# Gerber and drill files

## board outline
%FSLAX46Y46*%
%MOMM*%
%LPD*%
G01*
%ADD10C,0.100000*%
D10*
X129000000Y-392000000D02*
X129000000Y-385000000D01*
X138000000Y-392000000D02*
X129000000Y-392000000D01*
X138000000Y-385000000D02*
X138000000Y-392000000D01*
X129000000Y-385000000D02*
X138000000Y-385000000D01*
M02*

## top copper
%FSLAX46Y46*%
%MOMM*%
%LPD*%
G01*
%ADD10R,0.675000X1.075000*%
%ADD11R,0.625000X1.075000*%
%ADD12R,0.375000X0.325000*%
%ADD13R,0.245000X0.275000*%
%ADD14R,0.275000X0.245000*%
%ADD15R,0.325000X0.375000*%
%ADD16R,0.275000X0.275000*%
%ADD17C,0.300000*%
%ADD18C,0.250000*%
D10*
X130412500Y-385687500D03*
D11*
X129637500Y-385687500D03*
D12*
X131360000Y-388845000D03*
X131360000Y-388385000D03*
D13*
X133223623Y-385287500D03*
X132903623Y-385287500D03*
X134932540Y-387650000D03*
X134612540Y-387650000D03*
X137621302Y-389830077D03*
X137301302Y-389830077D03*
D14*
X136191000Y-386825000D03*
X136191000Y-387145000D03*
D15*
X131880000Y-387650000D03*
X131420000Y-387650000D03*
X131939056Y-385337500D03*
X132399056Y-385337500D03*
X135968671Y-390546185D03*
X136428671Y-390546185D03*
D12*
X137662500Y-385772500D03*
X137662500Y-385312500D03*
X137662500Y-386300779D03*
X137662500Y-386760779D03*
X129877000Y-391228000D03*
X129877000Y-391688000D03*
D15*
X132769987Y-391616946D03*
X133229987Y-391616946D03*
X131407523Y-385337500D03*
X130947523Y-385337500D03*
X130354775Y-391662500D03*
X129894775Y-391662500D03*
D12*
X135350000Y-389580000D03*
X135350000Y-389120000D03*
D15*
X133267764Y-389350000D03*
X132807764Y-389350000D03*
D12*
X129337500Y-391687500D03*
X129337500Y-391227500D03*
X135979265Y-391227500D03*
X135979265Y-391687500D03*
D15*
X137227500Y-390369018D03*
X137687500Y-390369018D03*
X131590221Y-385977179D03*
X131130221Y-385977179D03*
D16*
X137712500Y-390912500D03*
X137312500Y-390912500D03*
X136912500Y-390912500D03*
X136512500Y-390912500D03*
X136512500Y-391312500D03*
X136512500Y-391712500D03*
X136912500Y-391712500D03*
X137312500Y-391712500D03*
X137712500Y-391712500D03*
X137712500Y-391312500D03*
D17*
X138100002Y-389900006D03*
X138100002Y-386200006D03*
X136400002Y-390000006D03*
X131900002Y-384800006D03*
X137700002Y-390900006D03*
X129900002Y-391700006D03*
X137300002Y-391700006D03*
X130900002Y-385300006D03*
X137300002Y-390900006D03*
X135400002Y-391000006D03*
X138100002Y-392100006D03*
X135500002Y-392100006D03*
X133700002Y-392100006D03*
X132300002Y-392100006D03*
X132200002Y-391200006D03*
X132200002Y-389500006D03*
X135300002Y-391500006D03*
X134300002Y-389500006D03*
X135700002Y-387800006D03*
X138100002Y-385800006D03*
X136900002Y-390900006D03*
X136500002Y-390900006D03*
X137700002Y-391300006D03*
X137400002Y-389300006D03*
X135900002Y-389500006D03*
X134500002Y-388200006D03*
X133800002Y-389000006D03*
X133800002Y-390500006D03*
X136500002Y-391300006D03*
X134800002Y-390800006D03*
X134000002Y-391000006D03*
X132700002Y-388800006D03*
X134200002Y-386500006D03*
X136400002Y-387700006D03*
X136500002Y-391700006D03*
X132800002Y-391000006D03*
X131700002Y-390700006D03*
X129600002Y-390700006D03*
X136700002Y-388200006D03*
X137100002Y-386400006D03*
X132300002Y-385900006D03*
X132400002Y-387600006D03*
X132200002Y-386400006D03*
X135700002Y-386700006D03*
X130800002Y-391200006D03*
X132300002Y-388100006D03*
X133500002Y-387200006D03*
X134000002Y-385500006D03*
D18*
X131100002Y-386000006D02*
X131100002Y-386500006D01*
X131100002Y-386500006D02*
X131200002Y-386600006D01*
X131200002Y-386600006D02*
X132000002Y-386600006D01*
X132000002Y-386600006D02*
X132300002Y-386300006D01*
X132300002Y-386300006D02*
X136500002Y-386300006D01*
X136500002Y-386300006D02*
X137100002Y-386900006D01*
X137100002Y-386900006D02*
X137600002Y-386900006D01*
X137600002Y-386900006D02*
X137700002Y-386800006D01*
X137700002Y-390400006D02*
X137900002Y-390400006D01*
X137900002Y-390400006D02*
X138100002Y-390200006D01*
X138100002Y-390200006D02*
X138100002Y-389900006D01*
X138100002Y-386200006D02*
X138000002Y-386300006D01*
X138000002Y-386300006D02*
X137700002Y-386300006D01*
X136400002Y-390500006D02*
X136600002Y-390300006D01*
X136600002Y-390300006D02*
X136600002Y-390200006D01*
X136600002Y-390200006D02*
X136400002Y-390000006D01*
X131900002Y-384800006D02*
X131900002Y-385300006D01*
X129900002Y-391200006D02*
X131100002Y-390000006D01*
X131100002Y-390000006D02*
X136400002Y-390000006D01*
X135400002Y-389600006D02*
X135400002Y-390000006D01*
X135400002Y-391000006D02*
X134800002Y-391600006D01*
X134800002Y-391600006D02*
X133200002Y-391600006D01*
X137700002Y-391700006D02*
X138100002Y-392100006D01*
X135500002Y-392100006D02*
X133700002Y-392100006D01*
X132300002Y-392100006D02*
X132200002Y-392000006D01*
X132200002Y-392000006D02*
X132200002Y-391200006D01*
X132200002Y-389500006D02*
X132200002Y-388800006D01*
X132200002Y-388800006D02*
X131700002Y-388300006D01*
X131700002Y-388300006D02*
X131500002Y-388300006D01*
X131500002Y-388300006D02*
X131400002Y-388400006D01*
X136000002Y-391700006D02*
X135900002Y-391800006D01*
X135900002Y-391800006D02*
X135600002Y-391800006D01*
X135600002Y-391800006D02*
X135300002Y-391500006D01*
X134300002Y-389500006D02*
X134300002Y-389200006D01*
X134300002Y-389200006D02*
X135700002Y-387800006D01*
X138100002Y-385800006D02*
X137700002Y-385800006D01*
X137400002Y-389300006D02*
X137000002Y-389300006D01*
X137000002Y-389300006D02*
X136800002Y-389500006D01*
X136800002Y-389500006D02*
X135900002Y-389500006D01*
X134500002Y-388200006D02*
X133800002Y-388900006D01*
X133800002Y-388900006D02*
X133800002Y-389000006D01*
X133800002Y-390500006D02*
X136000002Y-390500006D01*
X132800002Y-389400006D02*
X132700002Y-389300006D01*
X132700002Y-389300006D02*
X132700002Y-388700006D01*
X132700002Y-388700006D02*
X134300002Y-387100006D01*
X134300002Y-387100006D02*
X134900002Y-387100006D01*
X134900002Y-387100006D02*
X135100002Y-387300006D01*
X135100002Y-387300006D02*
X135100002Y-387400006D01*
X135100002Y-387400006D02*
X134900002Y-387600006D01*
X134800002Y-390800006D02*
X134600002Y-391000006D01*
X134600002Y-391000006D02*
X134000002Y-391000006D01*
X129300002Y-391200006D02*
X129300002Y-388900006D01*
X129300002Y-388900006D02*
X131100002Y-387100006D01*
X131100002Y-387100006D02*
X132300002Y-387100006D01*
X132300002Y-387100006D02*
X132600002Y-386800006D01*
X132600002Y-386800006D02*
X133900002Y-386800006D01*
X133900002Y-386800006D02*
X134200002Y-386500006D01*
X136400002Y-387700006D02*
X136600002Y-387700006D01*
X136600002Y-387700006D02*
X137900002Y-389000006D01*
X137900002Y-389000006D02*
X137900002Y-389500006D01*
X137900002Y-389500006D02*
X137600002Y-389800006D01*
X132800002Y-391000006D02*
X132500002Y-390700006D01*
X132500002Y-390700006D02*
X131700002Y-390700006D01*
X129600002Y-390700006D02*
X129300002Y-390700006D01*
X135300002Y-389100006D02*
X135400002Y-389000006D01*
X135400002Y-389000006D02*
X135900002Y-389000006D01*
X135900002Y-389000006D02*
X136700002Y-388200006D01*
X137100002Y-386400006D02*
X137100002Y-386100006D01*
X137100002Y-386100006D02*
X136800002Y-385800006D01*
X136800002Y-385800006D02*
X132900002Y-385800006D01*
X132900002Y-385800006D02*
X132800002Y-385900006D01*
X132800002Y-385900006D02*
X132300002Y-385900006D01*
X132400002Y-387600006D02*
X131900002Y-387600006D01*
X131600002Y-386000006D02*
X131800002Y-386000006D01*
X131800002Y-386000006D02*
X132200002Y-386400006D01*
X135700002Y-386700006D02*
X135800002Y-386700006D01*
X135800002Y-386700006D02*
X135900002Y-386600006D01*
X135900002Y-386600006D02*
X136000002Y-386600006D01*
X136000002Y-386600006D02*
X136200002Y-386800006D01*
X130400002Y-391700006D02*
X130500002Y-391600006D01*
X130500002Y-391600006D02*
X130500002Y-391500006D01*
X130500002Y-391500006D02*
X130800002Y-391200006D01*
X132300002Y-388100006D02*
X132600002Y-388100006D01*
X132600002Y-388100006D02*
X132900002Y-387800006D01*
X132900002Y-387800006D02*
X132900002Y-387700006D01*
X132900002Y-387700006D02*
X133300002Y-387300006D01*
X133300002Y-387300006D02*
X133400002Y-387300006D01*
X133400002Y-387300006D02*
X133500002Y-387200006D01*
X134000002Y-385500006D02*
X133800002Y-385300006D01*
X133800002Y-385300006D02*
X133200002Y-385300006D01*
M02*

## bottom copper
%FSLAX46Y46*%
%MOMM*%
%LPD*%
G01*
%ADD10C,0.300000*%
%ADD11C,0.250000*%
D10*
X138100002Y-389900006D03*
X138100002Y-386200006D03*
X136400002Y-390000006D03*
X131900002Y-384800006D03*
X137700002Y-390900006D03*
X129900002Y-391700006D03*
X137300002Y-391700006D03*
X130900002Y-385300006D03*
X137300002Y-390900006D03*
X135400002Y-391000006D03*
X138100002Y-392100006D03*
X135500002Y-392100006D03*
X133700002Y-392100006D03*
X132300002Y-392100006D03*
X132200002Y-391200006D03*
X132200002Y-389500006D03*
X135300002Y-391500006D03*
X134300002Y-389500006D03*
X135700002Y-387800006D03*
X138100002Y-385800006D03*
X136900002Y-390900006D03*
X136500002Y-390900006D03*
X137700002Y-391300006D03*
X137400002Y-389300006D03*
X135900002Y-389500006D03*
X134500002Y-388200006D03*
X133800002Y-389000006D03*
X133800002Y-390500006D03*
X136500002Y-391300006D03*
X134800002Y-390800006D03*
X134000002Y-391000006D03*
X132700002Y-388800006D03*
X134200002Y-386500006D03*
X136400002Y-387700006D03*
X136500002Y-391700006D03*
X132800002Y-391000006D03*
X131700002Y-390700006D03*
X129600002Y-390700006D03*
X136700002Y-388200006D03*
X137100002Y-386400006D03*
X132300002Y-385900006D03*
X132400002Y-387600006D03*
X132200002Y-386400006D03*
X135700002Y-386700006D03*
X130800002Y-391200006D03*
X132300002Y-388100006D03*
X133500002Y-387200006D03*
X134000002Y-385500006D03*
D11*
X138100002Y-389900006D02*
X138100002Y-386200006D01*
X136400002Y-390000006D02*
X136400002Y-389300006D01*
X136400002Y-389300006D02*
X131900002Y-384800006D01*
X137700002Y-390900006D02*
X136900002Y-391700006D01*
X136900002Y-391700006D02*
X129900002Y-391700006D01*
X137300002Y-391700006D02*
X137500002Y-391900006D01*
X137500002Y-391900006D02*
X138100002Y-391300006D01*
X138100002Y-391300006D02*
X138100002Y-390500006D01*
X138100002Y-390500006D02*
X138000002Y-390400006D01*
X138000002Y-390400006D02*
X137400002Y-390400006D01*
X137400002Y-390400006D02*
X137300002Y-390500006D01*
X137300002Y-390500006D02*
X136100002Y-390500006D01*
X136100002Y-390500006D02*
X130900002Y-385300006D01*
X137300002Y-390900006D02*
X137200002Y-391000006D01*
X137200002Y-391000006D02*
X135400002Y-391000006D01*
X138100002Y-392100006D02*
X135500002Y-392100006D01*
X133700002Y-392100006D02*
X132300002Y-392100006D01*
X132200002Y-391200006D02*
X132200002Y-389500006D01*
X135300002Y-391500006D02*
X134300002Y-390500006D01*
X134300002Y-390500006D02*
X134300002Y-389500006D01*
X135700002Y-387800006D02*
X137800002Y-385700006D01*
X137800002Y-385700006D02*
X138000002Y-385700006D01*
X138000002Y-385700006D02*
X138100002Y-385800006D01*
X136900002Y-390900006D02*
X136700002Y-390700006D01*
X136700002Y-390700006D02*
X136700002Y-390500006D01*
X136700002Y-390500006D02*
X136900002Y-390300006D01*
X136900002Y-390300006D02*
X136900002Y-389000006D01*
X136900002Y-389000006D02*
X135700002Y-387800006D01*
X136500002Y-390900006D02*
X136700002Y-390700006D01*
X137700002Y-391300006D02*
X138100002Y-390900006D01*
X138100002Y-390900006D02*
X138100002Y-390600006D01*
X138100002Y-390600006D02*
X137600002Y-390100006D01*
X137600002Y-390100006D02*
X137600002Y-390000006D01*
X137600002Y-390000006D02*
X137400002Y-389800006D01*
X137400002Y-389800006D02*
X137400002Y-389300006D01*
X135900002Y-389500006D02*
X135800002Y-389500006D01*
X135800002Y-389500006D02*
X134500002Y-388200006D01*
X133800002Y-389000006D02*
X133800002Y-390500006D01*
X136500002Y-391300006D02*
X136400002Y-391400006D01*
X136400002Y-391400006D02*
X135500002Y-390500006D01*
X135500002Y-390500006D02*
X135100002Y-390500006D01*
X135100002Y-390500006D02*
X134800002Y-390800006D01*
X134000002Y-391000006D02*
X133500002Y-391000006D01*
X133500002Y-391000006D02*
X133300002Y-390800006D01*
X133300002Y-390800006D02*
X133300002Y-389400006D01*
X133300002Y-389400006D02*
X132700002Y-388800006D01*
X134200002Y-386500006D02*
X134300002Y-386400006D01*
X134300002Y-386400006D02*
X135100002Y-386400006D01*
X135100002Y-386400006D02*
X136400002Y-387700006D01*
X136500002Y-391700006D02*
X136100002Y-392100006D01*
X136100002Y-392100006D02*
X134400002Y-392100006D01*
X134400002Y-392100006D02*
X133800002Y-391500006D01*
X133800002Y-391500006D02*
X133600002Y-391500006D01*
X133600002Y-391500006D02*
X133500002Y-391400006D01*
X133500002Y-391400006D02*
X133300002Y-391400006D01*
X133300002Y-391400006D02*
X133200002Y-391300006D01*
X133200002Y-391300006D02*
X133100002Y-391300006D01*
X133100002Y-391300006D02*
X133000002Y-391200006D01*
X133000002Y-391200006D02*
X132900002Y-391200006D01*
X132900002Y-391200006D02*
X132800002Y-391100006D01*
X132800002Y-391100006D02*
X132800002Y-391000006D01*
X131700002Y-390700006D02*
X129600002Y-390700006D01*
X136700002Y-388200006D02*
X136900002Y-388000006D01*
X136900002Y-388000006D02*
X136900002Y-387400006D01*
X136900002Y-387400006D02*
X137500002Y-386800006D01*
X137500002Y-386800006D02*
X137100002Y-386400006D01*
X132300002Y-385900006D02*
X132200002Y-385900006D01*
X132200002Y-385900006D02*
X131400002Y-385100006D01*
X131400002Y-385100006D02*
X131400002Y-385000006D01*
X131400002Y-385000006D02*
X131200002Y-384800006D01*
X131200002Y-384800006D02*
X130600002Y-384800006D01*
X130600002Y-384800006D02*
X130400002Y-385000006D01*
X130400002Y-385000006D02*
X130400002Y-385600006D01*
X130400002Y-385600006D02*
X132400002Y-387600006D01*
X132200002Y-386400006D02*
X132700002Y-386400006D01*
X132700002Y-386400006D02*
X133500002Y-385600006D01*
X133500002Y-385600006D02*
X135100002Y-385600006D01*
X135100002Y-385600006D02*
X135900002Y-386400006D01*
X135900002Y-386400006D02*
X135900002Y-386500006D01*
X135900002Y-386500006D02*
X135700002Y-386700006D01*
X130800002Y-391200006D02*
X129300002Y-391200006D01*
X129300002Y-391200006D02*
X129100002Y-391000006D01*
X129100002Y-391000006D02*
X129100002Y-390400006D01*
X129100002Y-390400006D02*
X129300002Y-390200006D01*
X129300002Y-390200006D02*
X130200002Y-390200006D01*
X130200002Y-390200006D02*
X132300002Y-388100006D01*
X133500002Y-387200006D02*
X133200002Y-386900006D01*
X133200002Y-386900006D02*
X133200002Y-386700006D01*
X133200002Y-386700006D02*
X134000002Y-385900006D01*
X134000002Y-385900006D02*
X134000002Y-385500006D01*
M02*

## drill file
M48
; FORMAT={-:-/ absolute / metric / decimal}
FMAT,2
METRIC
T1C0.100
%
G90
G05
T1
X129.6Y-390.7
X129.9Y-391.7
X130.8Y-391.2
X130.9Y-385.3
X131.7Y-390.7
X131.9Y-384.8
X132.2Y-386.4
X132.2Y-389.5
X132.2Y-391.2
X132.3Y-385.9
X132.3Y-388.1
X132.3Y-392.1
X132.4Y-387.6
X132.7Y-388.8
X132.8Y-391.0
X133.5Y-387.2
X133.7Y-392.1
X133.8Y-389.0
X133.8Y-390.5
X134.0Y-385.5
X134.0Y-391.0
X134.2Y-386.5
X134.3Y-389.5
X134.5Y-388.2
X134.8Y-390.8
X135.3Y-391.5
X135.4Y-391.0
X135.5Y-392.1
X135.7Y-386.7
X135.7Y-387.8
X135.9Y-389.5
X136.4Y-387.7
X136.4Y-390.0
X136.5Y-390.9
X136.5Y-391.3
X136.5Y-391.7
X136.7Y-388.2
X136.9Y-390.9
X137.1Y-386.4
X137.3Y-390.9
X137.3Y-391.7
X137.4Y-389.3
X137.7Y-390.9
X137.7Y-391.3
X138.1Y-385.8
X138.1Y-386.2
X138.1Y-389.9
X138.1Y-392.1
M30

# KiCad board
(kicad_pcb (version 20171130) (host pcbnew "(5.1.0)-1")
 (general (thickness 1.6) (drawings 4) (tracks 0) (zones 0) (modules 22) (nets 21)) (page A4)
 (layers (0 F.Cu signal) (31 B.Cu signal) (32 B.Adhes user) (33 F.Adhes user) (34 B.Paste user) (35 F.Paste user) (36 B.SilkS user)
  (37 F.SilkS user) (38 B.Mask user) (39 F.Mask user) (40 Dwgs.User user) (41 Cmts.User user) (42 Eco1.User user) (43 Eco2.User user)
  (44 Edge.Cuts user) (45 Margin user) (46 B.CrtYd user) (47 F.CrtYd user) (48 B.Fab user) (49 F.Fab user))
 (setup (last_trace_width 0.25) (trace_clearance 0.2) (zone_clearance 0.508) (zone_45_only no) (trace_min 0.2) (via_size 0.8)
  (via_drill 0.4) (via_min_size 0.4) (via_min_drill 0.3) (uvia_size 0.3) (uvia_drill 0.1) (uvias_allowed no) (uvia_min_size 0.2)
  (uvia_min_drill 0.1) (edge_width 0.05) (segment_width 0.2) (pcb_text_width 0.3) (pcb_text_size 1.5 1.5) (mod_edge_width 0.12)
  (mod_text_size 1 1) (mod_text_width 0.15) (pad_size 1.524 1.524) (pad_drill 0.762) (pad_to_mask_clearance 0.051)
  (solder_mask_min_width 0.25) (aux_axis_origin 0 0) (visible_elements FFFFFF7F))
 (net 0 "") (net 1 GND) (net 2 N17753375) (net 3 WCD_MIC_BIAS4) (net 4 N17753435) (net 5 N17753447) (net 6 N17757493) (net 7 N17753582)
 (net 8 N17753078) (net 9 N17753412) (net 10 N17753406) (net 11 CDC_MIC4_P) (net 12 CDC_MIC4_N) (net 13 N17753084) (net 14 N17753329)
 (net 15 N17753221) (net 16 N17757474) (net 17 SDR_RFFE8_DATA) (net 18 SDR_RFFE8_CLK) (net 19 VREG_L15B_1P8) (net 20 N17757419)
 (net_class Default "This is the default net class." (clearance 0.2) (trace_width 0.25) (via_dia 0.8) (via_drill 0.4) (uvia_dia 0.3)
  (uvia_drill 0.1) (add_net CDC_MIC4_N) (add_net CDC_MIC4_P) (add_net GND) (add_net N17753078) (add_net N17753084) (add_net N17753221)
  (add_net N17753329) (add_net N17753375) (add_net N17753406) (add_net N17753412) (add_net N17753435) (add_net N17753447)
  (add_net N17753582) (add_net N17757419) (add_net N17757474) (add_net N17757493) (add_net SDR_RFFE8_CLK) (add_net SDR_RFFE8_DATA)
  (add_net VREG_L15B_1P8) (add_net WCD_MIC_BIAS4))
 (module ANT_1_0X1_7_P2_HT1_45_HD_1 (layer F.Cu) (at 129.862500 385.687500 270.000000)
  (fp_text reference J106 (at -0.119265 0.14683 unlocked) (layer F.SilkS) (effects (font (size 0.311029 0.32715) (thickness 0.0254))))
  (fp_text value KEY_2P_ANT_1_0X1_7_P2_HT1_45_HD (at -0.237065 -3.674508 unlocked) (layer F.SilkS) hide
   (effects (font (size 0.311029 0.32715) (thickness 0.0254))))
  (pad 1 smd rect (at 0 -0.55) (size 0.675 1.075) (layers F.Cu F.Mask F.Paste) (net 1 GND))
  (pad 2 smd rect (at 0 0.225) (size 0.625 1.075) (layers F.Cu F.Mask F.Paste) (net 1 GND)))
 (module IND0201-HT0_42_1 (layer F.Cu) (at 131.360000 388.615000 90.000000)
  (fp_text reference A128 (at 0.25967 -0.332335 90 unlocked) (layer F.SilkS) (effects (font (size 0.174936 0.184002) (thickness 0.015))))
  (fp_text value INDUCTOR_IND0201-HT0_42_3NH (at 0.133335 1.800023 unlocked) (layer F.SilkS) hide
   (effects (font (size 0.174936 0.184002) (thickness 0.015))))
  (pad 1 smd rect (at -0.23 0) (size 0.375 0.325) (layers F.Cu F.Mask F.Paste) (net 1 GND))
  (pad 2 smd rect (at 0.23 0) (size 0.375 0.325) (layers F.Cu F.Mask F.Paste) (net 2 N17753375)))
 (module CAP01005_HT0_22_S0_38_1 (layer F.Cu) (at 133.063623 385.287500 180.000000)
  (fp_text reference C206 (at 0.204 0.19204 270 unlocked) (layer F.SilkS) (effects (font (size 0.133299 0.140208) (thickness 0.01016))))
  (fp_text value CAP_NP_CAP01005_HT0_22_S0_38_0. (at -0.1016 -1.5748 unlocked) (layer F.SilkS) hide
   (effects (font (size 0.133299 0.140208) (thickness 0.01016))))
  (pad 1 smd rect (at -0.16 0 270.000000) (size 0.275 0.245) (layers F.Cu F.Mask F.Paste) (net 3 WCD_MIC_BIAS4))
  (pad 2 smd rect (at 0.16 0 270.000000) (size 0.275 0.245) (layers F.Cu F.Mask F.Paste) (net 1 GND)))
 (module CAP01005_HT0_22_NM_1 (layer F.Cu) (at 134.772540 387.650000 180.000000)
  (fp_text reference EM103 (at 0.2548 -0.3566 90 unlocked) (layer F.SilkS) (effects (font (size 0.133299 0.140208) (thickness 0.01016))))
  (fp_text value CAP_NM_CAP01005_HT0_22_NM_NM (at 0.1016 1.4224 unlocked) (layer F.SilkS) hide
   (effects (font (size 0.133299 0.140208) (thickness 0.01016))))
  (pad 1 smd rect (at -0.16 0 90.000000) (size 0.275 0.245) (layers F.Cu F.Mask F.Paste) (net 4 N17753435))
  (pad 2 smd rect (at 0.16 0 90.000000) (size 0.275 0.245) (layers F.Cu F.Mask F.Paste) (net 1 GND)))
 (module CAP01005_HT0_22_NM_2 (layer F.Cu) (at 137.461302 389.830077 180.000000)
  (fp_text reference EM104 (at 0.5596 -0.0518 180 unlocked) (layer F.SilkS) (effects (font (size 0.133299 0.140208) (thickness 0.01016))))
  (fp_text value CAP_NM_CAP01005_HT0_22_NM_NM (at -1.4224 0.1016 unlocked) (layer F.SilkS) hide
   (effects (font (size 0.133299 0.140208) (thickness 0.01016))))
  (pad 1 smd rect (at -0.16 0) (size 0.245 0.275) (layers F.Cu F.Mask F.Paste) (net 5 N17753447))
  (pad 2 smd rect (at 0.16 0) (size 0.245 0.275) (layers F.Cu F.Mask F.Paste) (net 1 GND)))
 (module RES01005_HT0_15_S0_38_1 (layer F.Cu) (at 136.191000 386.985000 270.000000)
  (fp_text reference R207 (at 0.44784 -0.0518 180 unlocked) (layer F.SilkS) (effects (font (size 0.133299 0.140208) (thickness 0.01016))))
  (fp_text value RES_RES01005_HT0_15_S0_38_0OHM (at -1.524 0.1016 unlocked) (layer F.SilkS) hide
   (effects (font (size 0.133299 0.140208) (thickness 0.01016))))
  (pad 1 smd rect (at -0.16 0 90.000000) (size 0.245 0.275) (layers F.Cu F.Mask F.Paste) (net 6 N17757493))
  (pad 2 smd rect (at 0.16 0 90.000000) (size 0.245 0.275) (layers F.Cu F.Mask F.Paste) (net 1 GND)))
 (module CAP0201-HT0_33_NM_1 (layer F.Cu) (at 131.650000 387.650000 180.000000)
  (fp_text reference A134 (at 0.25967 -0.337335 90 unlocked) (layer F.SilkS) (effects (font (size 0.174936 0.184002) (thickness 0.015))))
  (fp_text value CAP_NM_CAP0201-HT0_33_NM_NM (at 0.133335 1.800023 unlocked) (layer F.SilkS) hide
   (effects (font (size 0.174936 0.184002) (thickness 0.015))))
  (pad 1 smd rect (at -0.23 0 90.000000) (size 0.375 0.325) (layers F.Cu F.Mask F.Paste) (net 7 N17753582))
  (pad 2 smd rect (at 0.23 0 90.000000) (size 0.375 0.325) (layers F.Cu F.Mask F.Paste) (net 1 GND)))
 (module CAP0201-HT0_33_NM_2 (layer F.Cu) (at 132.169056 385.337500)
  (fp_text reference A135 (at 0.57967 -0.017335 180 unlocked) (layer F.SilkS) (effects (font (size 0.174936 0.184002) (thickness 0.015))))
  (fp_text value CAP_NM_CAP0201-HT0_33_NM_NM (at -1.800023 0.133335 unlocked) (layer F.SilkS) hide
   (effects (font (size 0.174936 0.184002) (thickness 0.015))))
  (pad 1 smd rect (at -0.23 0 180.000000) (size 0.325 0.375) (layers F.Cu F.Mask F.Paste) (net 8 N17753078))
  (pad 2 smd rect (at 0.23 0 180.000000) (size 0.325 0.375) (layers F.Cu F.Mask F.Paste) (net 1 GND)))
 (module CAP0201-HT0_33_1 (layer F.Cu) (at 136.198671 390.546185)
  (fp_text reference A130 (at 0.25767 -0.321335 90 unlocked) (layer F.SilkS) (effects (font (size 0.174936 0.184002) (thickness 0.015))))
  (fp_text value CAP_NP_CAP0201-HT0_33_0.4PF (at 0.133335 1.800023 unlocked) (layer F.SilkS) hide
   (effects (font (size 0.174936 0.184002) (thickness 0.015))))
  (pad 1 smd rect (at -0.23 0 270.000000) (size 0.375 0.325) (layers F.Cu F.Mask F.Paste) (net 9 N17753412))
  (pad 2 smd rect (at 0.23 0 270.000000) (size 0.375 0.325) (layers F.Cu F.Mask F.Paste) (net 8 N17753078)))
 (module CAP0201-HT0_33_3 (layer F.Cu) (at 137.662500 385.542500 90.000000)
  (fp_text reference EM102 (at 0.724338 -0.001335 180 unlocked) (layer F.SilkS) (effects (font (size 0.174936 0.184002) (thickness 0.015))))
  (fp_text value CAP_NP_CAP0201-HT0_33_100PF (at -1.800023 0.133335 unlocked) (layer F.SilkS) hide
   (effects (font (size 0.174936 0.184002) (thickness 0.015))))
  (pad 1 smd rect (at -0.23 0 270.000000) (size 0.325 0.375) (layers F.Cu F.Mask F.Paste) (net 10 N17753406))
  (pad 2 smd rect (at 0.23 0 270.000000) (size 0.325 0.375) (layers F.Cu F.Mask F.Paste) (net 1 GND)))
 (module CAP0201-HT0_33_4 (layer F.Cu) (at 137.662500 386.530779 270.000000)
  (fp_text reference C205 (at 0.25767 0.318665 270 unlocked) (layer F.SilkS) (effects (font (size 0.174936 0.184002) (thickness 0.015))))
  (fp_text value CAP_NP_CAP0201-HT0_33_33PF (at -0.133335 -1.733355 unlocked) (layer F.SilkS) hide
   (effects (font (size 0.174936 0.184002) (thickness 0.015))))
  (pad 1 smd rect (at -0.23 0) (size 0.375 0.325) (layers F.Cu F.Mask F.Paste) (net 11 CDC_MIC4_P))
  (pad 2 smd rect (at 0.23 0) (size 0.375 0.325) (layers F.Cu F.Mask F.Paste) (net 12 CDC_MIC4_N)))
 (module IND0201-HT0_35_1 (layer F.Cu) (at 129.877000 391.458000 270.000000)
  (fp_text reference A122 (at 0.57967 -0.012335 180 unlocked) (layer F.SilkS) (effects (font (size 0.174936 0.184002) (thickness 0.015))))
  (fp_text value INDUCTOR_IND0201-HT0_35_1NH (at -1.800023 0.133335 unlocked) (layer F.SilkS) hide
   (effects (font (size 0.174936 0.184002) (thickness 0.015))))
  (pad 1 smd rect (at -0.23 0 90.000000) (size 0.325 0.375) (layers F.Cu F.Mask F.Paste) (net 8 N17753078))
  (pad 2 smd rect (at 0.23 0 90.000000) (size 0.325 0.375) (layers F.Cu F.Mask F.Paste) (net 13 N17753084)))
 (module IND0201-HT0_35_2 (layer F.Cu) (at 132.999987 391.616946)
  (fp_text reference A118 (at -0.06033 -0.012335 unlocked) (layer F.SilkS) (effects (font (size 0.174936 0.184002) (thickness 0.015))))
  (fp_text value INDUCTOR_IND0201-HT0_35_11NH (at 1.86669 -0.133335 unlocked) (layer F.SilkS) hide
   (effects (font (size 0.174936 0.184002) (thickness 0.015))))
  (pad 1 smd rect (at -0.23 0) (size 0.325 0.375) (layers F.Cu F.Mask F.Paste) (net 1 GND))
  (pad 2 smd rect (at 0.23 0) (size 0.325 0.375) (layers F.Cu F.Mask F.Paste) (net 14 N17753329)))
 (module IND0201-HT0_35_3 (layer F.Cu) (at 131.177523 385.337500 180.000000)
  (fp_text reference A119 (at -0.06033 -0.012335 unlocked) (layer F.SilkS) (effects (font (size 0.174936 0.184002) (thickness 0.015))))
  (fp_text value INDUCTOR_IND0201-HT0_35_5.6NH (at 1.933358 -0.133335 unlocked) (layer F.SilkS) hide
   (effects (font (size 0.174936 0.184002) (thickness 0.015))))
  (pad 1 smd rect (at -0.23 0 180.000000) (size 0.325 0.375) (layers F.Cu F.Mask F.Paste) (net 1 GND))
  (pad 2 smd rect (at 0.23 0 180.000000) (size 0.325 0.375) (layers F.Cu F.Mask F.Paste) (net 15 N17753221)))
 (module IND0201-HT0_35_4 (layer F.Cu) (at 130.124775 391.662500 180.000000)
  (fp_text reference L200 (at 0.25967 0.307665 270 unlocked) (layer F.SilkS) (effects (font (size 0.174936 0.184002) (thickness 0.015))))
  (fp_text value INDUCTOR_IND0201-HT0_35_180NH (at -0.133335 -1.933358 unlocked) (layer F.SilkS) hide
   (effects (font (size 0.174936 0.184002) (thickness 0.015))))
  (pad 1 smd rect (at -0.23 0 270.000000) (size 0.375 0.325) (layers F.Cu F.Mask F.Paste) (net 3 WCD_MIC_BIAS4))
  (pad 2 smd rect (at 0.23 0 270.000000) (size 0.375 0.325) (layers F.Cu F.Mask F.Paste) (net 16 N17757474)))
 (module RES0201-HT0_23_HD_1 (layer F.Cu) (at 135.350000 389.350000 90.000000)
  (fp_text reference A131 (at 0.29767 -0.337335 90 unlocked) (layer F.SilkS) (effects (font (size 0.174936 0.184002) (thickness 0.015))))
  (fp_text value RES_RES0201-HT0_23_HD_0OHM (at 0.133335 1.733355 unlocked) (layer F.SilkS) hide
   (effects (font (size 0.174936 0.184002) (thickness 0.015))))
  (pad 1 smd rect (at -0.23 0) (size 0.375 0.325) (layers F.Cu F.Mask F.Paste) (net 8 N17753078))
  (pad 2 smd rect (at 0.23 0) (size 0.375 0.325) (layers F.Cu F.Mask F.Paste) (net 7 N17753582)))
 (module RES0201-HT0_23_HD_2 (layer F.Cu) (at 133.037764 389.350000 180.000000)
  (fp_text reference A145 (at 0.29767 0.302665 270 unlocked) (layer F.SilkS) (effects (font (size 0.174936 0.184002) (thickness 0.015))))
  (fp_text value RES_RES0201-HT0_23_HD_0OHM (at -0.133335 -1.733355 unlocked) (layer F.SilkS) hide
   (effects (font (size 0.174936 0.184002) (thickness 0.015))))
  (pad 1 smd rect (at -0.23 0 270.000000) (size 0.375 0.325) (layers F.Cu F.Mask F.Paste) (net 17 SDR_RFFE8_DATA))
  (pad 2 smd rect (at 0.23 0 270.000000) (size 0.375 0.325) (layers F.Cu F.Mask F.Paste) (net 4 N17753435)))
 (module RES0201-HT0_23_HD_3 (layer F.Cu) (at 129.337500 391.457500 90.000000)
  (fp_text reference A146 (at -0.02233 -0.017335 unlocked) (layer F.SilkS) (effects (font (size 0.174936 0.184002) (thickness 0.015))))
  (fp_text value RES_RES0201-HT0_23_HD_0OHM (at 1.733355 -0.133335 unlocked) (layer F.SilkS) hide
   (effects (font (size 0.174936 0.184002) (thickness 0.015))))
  (pad 1 smd rect (at -0.23 0 90.000000) (size 0.325 0.375) (layers F.Cu F.Mask F.Paste) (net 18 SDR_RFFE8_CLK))
  (pad 2 smd rect (at 0.23 0 90.000000) (size 0.325 0.375) (layers F.Cu F.Mask F.Paste) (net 5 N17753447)))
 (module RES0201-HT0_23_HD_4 (layer F.Cu) (at 135.979265 391.457500 270.000000)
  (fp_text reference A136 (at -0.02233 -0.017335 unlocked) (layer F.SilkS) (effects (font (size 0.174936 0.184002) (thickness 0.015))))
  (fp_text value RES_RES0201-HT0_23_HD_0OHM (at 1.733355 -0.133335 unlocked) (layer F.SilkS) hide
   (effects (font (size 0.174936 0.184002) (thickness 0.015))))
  (pad 1 smd rect (at -0.23 0 270.000000) (size 0.325 0.375) (layers F.Cu F.Mask F.Paste) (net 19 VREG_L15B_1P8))
  (pad 2 smd rect (at 0.23 0 270.000000) (size 0.325 0.375) (layers F.Cu F.Mask F.Paste) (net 10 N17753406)))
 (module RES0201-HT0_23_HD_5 (layer F.Cu) (at 137.457500 390.369018)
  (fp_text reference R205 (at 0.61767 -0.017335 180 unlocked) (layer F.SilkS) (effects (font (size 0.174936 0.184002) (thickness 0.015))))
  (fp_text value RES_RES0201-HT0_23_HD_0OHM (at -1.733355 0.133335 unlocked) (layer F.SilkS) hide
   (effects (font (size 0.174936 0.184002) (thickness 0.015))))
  (pad 1 smd rect (at -0.23 0 180.000000) (size 0.325 0.375) (layers F.Cu F.Mask F.Paste) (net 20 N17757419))
  (pad 2 smd rect (at 0.23 0 180.000000) (size 0.325 0.375) (layers F.Cu F.Mask F.Paste) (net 11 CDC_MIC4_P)))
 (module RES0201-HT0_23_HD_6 (layer F.Cu) (at 131.360221 385.977179 180.000000)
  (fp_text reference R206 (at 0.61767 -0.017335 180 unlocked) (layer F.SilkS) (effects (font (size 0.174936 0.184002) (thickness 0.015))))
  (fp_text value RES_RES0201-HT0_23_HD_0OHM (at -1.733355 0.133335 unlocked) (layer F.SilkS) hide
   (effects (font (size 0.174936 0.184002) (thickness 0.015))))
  (pad 1 smd rect (at -0.23 0) (size 0.325 0.375) (layers F.Cu F.Mask F.Paste) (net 6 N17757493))
  (pad 2 smd rect (at 0.23 0) (size 0.325 0.375) (layers F.Cu F.Mask F.Paste) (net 12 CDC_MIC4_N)))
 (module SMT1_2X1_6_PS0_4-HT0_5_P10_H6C (layer F.Cu) (at 137.112500 391.312500 180.000000)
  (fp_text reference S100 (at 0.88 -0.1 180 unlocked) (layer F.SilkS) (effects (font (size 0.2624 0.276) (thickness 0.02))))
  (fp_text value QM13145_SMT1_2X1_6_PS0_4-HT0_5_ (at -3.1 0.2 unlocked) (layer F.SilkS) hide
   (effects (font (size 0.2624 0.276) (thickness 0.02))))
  (pad 1 smd rect (at -0.6 0.4) (size 0.275 0.275) (layers F.Cu F.Mask F.Paste) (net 13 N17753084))
  (pad 2 smd rect (at -0.2 0.4) (size 0.275 0.275) (layers F.Cu F.Mask F.Paste) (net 14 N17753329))
  (pad 3 smd rect (at 0.2 0.4) (size 0.275 0.275) (layers F.Cu F.Mask F.Paste) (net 10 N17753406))
  (pad 4 smd rect (at 0.6 0.4) (size 0.275 0.275) (layers F.Cu F.Mask F.Paste) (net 10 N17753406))
  (pad 5 smd rect (at 0.6 0) (size 0.275 0.275) (layers F.Cu F.Mask F.Paste) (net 4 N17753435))
  (pad 6 smd rect (at 0.6 -0.4) (size 0.275 0.275) (layers F.Cu F.Mask F.Paste) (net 5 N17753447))
  (pad 7 smd rect (at 0.2 -0.4) (size 0.275 0.275) (layers F.Cu F.Mask F.Paste) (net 1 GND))
  (pad 8 smd rect (at -0.2 -0.4) (size 0.275 0.275) (layers F.Cu F.Mask F.Paste) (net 15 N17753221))
  (pad 9 smd rect (at -0.6 -0.4) (size 0.275 0.275) (layers F.Cu F.Mask F.Paste) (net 2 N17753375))
  (pad 10 smd rect (at -0.6 0) (size 0.275 0.275) (layers F.Cu F.Mask F.Paste) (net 9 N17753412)))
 (gr_line (start 129 392) (end 129 385) (layer Edge.Cuts) (width 0.1))
 (gr_line (start 138 392) (end 129 392) (layer Edge.Cuts) (width 0.1))
 (gr_line (start 138 385) (end 138 392) (layer Edge.Cuts) (width 0.1))
 (gr_line (start 129 385) (end 138 385) (layer Edge.Cuts) (width 0.1))
 (segment (start 131.100002 386.000006) (end 131.100002 386.500006) (width 0.250000) (layer F.Cu) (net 12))
 (segment (start 131.100002 386.500006) (end 131.200002 386.600006) (width 0.250000) (layer F.Cu) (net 12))
 (segment (start 131.200002 386.600006) (end 132.000002 386.600006) (width 0.250000) (layer F.Cu) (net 12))
 (segment (start 132.000002 386.600006) (end 132.300002 386.300006) (width 0.250000) (layer F.Cu) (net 12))
 (segment (start 132.300002 386.300006) (end 136.500002 386.300006) (width 0.250000) (layer F.Cu) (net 12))
 (segment (start 136.500002 386.300006) (end 137.100002 386.900006) (width 0.250000) (layer F.Cu) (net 12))
 (segment (start 137.100002 386.900006) (end 137.600002 386.900006) (width 0.250000) (layer F.Cu) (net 12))
 (segment (start 137.600002 386.900006) (end 137.700002 386.800006) (width 0.250000) (layer F.Cu) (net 12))
 (segment (start 137.700002 390.400006) (end 137.900002 390.400006) (width 0.250000) (layer F.Cu) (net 11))
 (segment (start 137.900002 390.400006) (end 138.100002 390.200006) (width 0.250000) (layer F.Cu) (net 11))
 (segment (start 138.100002 390.200006) (end 138.100002 389.900006) (width 0.250000) (layer F.Cu) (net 11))
 (segment (start 138.100002 389.900006) (end 138.100002 386.200006) (width 0.250000) (layer B.Cu) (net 11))
 (segment (start 138.100002 386.200006) (end 138.000002 386.300006) (width 0.250000) (layer F.Cu) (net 11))
 (segment (start 138.000002 386.300006) (end 137.700002 386.300006) (width 0.250000) (layer F.Cu) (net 11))
 (via micro (at 138.100002 389.900006) (size 0.300000) (drill 0.100000) (layers F.Cu B.Cu) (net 11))
 (via micro (at 138.100002 386.200006) (size 0.300000) (drill 0.100000) (layers F.Cu B.Cu) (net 11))
 (segment (start 136.400002 390.500006) (end 136.600002 390.300006) (width 0.250000) (layer F.Cu) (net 8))
 (segment (start 136.600002 390.300006) (end 136.600002 390.200006) (width 0.250000) (layer F.Cu) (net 8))
 (segment (start 136.600002 390.200006) (end 136.400002 390.000006) (width 0.250000) (layer F.Cu) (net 8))
 (segment (start 136.400002 390.000006) (end 136.400002 389.300006) (width 0.250000) (layer B.Cu) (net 8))
 (segment (start 136.400002 389.300006) (end 131.900002 384.800006) (width 0.250000) (layer B.Cu) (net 8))
 (segment (start 131.900002 384.800006) (end 131.900002 385.300006) (width 0.250000) (layer F.Cu) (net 8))
 (segment (start 129.900002 391.200006) (end 131.100002 390.000006) (width 0.250000) (layer F.Cu) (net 8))
 (segment (start 131.100002 390.000006) (end 136.400002 390.000006) (width 0.250000) (layer F.Cu) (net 8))
 (segment (start 135.400002 389.600006) (end 135.400002 390.000006) (width 0.250000) (layer F.Cu) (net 8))
 (via micro (at 136.400002 390.000006) (size 0.300000) (drill 0.100000) (layers F.Cu B.Cu) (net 8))
 (via micro (at 131.900002 384.800006) (size 0.300000) (drill 0.100000) (layers F.Cu B.Cu) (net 8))
 (segment (start 137.700002 390.900006) (end 136.900002 391.700006) (width 0.250000) (layer B.Cu) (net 13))
 (segment (start 136.900002 391.700006) (end 129.900002 391.700006) (width 0.250000) (layer B.Cu) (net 13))
 (via micro (at 137.700002 390.900006) (size 0.300000) (drill 0.100000) (layers F.Cu B.Cu) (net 13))
 (via micro (at 129.900002 391.700006) (size 0.300000) (drill 0.100000) (layers F.Cu B.Cu) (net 13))
 (segment (start 137.300002 391.700006) (end 137.500002 391.900006) (width 0.250000) (layer B.Cu) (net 15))
 (segment (start 137.500002 391.900006) (end 138.100002 391.300006) (width 0.250000) (layer B.Cu) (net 15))
 (segment (start 138.100002 391.300006) (end 138.100002 390.500006) (width 0.250000) (layer B.Cu) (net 15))
 (segment (start 138.100002 390.500006) (end 138.000002 390.400006) (width 0.250000) (layer B.Cu) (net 15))
 (segment (start 138.000002 390.400006) (end 137.400002 390.400006) (width 0.250000) (layer B.Cu) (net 15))
 (segment (start 137.400002 390.400006) (end 137.300002 390.500006) (width 0.250000) (layer B.Cu) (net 15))
 (segment (start 137.300002 390.500006) (end 136.100002 390.500006) (width 0.250000) (layer B.Cu) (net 15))
 (segment (start 136.100002 390.500006) (end 130.900002 385.300006) (width 0.250000) (layer B.Cu) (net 15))
 (via micro (at 137.300002 391.700006) (size 0.300000) (drill 0.100000) (layers F.Cu B.Cu) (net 15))
 (via micro (at 130.900002 385.300006) (size 0.300000) (drill 0.100000) (layers F.Cu B.Cu) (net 15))
 (segment (start 137.300002 390.900006) (end 137.200002 391.000006) (width 0.250000) (layer B.Cu) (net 14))
 (segment (start 137.200002 391.000006) (end 135.400002 391.000006) (width 0.250000) (layer B.Cu) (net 14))
 (segment (start 135.400002 391.000006) (end 134.800002 391.600006) (width 0.250000) (layer F.Cu) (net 14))
 (segment (start 134.800002 391.600006) (end 133.200002 391.600006) (width 0.250000) (layer F.Cu) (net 14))
 (via micro (at 137.300002 390.900006) (size 0.300000) (drill 0.100000) (layers F.Cu B.Cu) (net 14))
 (via micro (at 135.400002 391.000006) (size 0.300000) (drill 0.100000) (layers F.Cu B.Cu) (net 14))
 (segment (start 137.700002 391.700006) (end 138.100002 392.100006) (width 0.250000) (layer F.Cu) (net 2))
 (segment (start 138.100002 392.100006) (end 135.500002 392.100006) (width 0.250000) (layer B.Cu) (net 2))
 (segment (start 135.500002 392.100006) (end 133.700002 392.100006) (width 0.250000) (layer F.Cu) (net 2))
 (segment (start 133.700002 392.100006) (end 132.300002 392.100006) (width 0.250000) (layer B.Cu) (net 2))
 (segment (start 132.300002 392.100006) (end 132.200002 392.000006) (width 0.250000) (layer F.Cu) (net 2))
 (segment (start 132.200002 392.000006) (end 132.200002 391.200006) (width 0.250000) (layer F.Cu) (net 2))
 (segment (start 132.200002 391.200006) (end 132.200002 389.500006) (width 0.250000) (layer B.Cu) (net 2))
 (segment (start 132.200002 389.500006) (end 132.200002 388.800006) (width 0.250000) (layer F.Cu) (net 2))
 (segment (start 132.200002 388.800006) (end 131.700002 388.300006) (width 0.250000) (layer F.Cu) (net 2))
 (segment (start 131.700002 388.300006) (end 131.500002 388.300006) (width 0.250000) (layer F.Cu) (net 2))
 (segment (start 131.500002 388.300006) (end 131.400002 388.400006) (width 0.250000) (layer F.Cu) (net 2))
 (via micro (at 138.100002 392.100006) (size 0.300000) (drill 0.100000) (layers F.Cu B.Cu) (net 2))
 (via micro (at 135.500002 392.100006) (size 0.300000) (drill 0.100000) (layers F.Cu B.Cu) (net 2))
 (via micro (at 133.700002 392.100006) (size 0.300000) (drill 0.100000) (layers F.Cu B.Cu) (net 2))
 (via micro (at 132.300002 392.100006) (size 0.300000) (drill 0.100000) (layers F.Cu B.Cu) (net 2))
 (via micro (at 132.200002 391.200006) (size 0.300000) (drill 0.100000) (layers F.Cu B.Cu) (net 2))
 (via micro (at 132.200002 389.500006) (size 0.300000) (drill 0.100000) (layers F.Cu B.Cu) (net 2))
 (segment (start 136.000002 391.700006) (end 135.900002 391.800006) (width 0.250000) (layer F.Cu) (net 10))
 (segment (start 135.900002 391.800006) (end 135.600002 391.800006) (width 0.250000) (layer F.Cu) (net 10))
 (segment (start 135.600002 391.800006) (end 135.300002 391.500006) (width 0.250000) (layer F.Cu) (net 10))
 (segment (start 135.300002 391.500006) (end 134.300002 390.500006) (width 0.250000) (layer B.Cu) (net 10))
 (segment (start 134.300002 390.500006) (end 134.300002 389.500006) (width 0.250000) (layer B.Cu) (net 10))
 (segment (start 134.300002 389.500006) (end 134.300002 389.200006) (width 0.250000) (layer F.Cu) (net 10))
 (segment (start 134.300002 389.200006) (end 135.700002 387.800006) (width 0.250000) (layer F.Cu) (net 10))
 (segment (start 135.700002 387.800006) (end 137.800002 385.700006) (width 0.250000) (layer B.Cu) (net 10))
 (segment (start 137.800002 385.700006) (end 138.000002 385.700006) (width 0.250000) (layer B.Cu) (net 10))
 (segment (start 138.000002 385.700006) (end 138.100002 385.800006) (width 0.250000) (layer B.Cu) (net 10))
 (segment (start 138.100002 385.800006) (end 137.700002 385.800006) (width 0.250000) (layer F.Cu) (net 10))
 (segment (start 136.900002 390.900006) (end 136.700002 390.700006) (width 0.250000) (layer B.Cu) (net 10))
 (segment (start 136.700002 390.700006) (end 136.700002 390.500006) (width 0.250000) (layer B.Cu) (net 10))
 (segment (start 136.700002 390.500006) (end 136.900002 390.300006) (width 0.250000) (layer B.Cu) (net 10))
 (segment (start 136.900002 390.300006) (end 136.900002 389.000006) (width 0.250000) (layer B.Cu) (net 10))
 (segment (start 136.900002 389.000006) (end 135.700002 387.800006) (width 0.250000) (layer B.Cu) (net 10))
 (segment (start 136.500002 390.900006) (end 136.700002 390.700006) (width 0.250000) (layer B.Cu) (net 10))
 (via micro (at 135.300002 391.500006) (size 0.300000) (drill 0.100000) (layers F.Cu B.Cu) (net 10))
 (via micro (at 134.300002 389.500006) (size 0.300000) (drill 0.100000) (layers F.Cu B.Cu) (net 10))
 (via micro (at 135.700002 387.800006) (size 0.300000) (drill 0.100000) (layers F.Cu B.Cu) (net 10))
 (via micro (at 138.100002 385.800006) (size 0.300000) (drill 0.100000) (layers F.Cu B.Cu) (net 10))
 (via micro (at 136.900002 390.900006) (size 0.300000) (drill 0.100000) (layers F.Cu B.Cu) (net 10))
 (via micro (at 136.500002 390.900006) (size 0.300000) (drill 0.100000) (layers F.Cu B.Cu) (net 10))
 (segment (start 137.700002 391.300006) (end 138.100002 390.900006) (width 0.250000) (layer B.Cu) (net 9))
 (segment (start 138.100002 390.900006) (end 138.100002 390.600006) (width 0.250000) (layer B.Cu) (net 9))
 (segment (start 138.100002 390.600006) (end 137.600002 390.100006) (width 0.250000) (layer B.Cu) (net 9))
 (segment (start 137.600002 390.100006) (end 137.600002 390.000006) (width 0.250000) (layer B.Cu) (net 9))
 (segment (start 137.600002 390.000006) (end 137.400002 389.800006) (width 0.250000) (layer B.Cu) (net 9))
 (segment (start 137.400002 389.800006) (end 137.400002 389.300006) (width 0.250000) (layer B.Cu) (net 9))
 (segment (start 137.400002 389.300006) (end 137.000002 389.300006) (width 0.250000) (layer F.Cu) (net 9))
 (segment (start 137.000002 389.300006) (end 136.800002 389.500006) (width 0.250000) (layer F.Cu) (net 9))
 (segment (start 136.800002 389.500006) (end 135.900002 389.500006) (width 0.250000) (layer F.Cu) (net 9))
 (segment (start 135.900002 389.500006) (end 135.800002 389.500006) (width 0.250000) (layer B.Cu) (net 9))
 (segment (start 135.800002 389.500006) (end 134.500002 388.200006) (width 0.250000) (layer B.Cu) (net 9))
 (segment (start 134.500002 388.200006) (end 133.800002 388.900006) (width 0.250000) (layer F.Cu) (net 9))
 (segment (start 133.800002 388.900006) (end 133.800002 389.000006) (width 0.250000) (layer F.Cu) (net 9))
 (segment (start 133.800002 389.000006) (end 133.800002 390.500006) (width 0.250000) (layer B.Cu) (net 9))
 (segment (start 133.800002 390.500006) (end 136.000002 390.500006) (width 0.250000) (layer F.Cu) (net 9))
 (via micro (at 137.700002 391.300006) (size 0.300000) (drill 0.100000) (layers F.Cu B.Cu) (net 9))
 (via micro (at 137.400002 389.300006) (size 0.300000) (drill 0.100000) (layers F.Cu B.Cu) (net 9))
 (via micro (at 135.900002 389.500006) (size 0.300000) (drill 0.100000) (layers F.Cu B.Cu) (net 9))
 (via micro (at 134.500002 388.200006) (size 0.300000) (drill 0.100000) (layers F.Cu B.Cu) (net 9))
 (via micro (at 133.800002 389.000006) (size 0.300000) (drill 0.100000) (layers F.Cu B.Cu) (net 9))
 (via micro (at 133.800002 390.500006) (size 0.300000) (drill 0.100000) (layers F.Cu B.Cu) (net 9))
 (segment (start 132.800002 389.400006) (end 132.700002 389.300006) (width 0.250000) (layer F.Cu) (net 4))
 (segment (start 132.700002 389.300006) (end 132.700002 388.700006) (width 0.250000) (layer F.Cu) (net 4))
 (segment (start 132.700002 388.700006) (end 134.300002 387.100006) (width 0.250000) (layer F.Cu) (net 4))
 (segment (start 134.300002 387.100006) (end 134.900002 387.100006) (width 0.250000) (layer F.Cu) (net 4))
 (segment (start 134.900002 387.100006) (end 135.100002 387.300006) (width 0.250000) (layer F.Cu) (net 4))
 (segment (start 135.100002 387.300006) (end 135.100002 387.400006) (width 0.250000) (layer F.Cu) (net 4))
 (segment (start 135.100002 387.400006) (end 134.900002 387.600006) (width 0.250000) (layer F.Cu) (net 4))
 (segment (start 136.500002 391.300006) (end 136.400002 391.400006) (width 0.250000) (layer B.Cu) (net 4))
 (segment (start 136.400002 391.400006) (end 135.500002 390.500006) (width 0.250000) (layer B.Cu) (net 4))
 (segment (start 135.500002 390.500006) (end 135.100002 390.500006) (width 0.250000) (layer B.Cu) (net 4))
 (segment (start 135.100002 390.500006) (end 134.800002 390.800006) (width 0.250000) (layer B.Cu) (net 4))
 (segment (start 134.800002 390.800006) (end 134.600002 391.000006) (width 0.250000) (layer F.Cu) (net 4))
 (segment (start 134.600002 391.000006) (end 134.000002 391.000006) (width 0.250000) (layer F.Cu) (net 4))
 (segment (start 134.000002 391.000006) (end 133.500002 391.000006) (width 0.250000) (layer B.Cu) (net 4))
 (segment (start 133.500002 391.000006) (end 133.300002 390.800006) (width 0.250000) (layer B.Cu) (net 4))
 (segment (start 133.300002 390.800006) (end 133.300002 389.400006) (width 0.250000) (layer B.Cu) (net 4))
 (segment (start 133.300002 389.400006) (end 132.700002 388.800006) (width 0.250000) (layer B.Cu) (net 4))
 (via micro (at 136.500002 391.300006) (size 0.300000) (drill 0.100000) (layers F.Cu B.Cu) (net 4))
 (via micro (at 134.800002 390.800006) (size 0.300000) (drill 0.100000) (layers F.Cu B.Cu) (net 4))
 (via micro (at 134.000002 391.000006) (size 0.300000) (drill 0.100000) (layers F.Cu B.Cu) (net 4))
 (via micro (at 132.700002 388.800006) (size 0.300000) (drill 0.100000) (layers F.Cu B.Cu) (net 4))
 (segment (start 129.300002 391.200006) (end 129.300002 388.900006) (width 0.250000) (layer F.Cu) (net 5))
 (segment (start 129.300002 388.900006) (end 131.100002 387.100006) (width 0.250000) (layer F.Cu) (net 5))
 (segment (start 131.100002 387.100006) (end 132.300002 387.100006) (width 0.250000) (layer F.Cu) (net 5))
 (segment (start 132.300002 387.100006) (end 132.600002 386.800006) (width 0.250000) (layer F.Cu) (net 5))
 (segment (start 132.600002 386.800006) (end 133.900002 386.800006) (width 0.250000) (layer F.Cu) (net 5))
 (segment (start 133.900002 386.800006) (end 134.200002 386.500006) (width 0.250000) (layer F.Cu) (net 5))
 (segment (start 134.200002 386.500006) (end 134.300002 386.400006) (width 0.250000) (layer B.Cu) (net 5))
 (segment (start 134.300002 386.400006) (end 135.100002 386.400006) (width 0.250000) (layer B.Cu) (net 5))
 (segment (start 135.100002 386.400006) (end 136.400002 387.700006) (width 0.250000) (layer B.Cu) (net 5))
 (segment (start 136.400002 387.700006) (end 136.600002 387.700006) (width 0.250000) (layer F.Cu) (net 5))
 (segment (start 136.600002 387.700006) (end 137.900002 389.000006) (width 0.250000) (layer F.Cu) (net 5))
 (segment (start 137.900002 389.000006) (end 137.900002 389.500006) (width 0.250000) (layer F.Cu) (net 5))
 (segment (start 137.900002 389.500006) (end 137.600002 389.800006) (width 0.250000) (layer F.Cu) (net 5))
 (segment (start 136.500002 391.700006) (end 136.100002 392.100006) (width 0.250000) (layer B.Cu) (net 5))
 (segment (start 136.100002 392.100006) (end 134.400002 392.100006) (width 0.250000) (layer B.Cu) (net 5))
 (segment (start 134.400002 392.100006) (end 133.800002 391.500006) (width 0.250000) (layer B.Cu) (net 5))
 (segment (start 133.800002 391.500006) (end 133.600002 391.500006) (width 0.250000) (layer B.Cu) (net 5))
 (segment (start 133.600002 391.500006) (end 133.500002 391.400006) (width 0.250000) (layer B.Cu) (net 5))
 (segment (start 133.500002 391.400006) (end 133.300002 391.400006) (width 0.250000) (layer B.Cu) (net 5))
 (segment (start 133.300002 391.400006) (end 133.200002 391.300006) (width 0.250000) (layer B.Cu) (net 5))
 (segment (start 133.200002 391.300006) (end 133.100002 391.300006) (width 0.250000) (layer B.Cu) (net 5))
 (segment (start 133.100002 391.300006) (end 133.000002 391.200006) (width 0.250000) (layer B.Cu) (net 5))
 (segment (start 133.000002 391.200006) (end 132.900002 391.200006) (width 0.250000) (layer B.Cu) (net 5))
 (segment (start 132.900002 391.200006) (end 132.800002 391.100006) (width 0.250000) (layer B.Cu) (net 5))
 (segment (start 132.800002 391.100006) (end 132.800002 391.000006) (width 0.250000) (layer B.Cu) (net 5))
 (segment (start 132.800002 391.000006) (end 132.500002 390.700006) (width 0.250000) (layer F.Cu) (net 5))
 (segment (start 132.500002 390.700006) (end 131.700002 390.700006) (width 0.250000) (layer F.Cu) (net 5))
 (segment (start 131.700002 390.700006) (end 129.600002 390.700006) (width 0.250000) (layer B.Cu) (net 5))
 (segment (start 129.600002 390.700006) (end 129.300002 390.700006) (width 0.250000) (layer F.Cu) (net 5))
 (via micro (at 134.200002 386.500006) (size 0.300000) (drill 0.100000) (layers F.Cu B.Cu) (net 5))
 (via micro (at 136.400002 387.700006) (size 0.300000) (drill 0.100000) (layers F.Cu B.Cu) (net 5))
 (via micro (at 136.500002 391.700006) (size 0.300000) (drill 0.100000) (layers F.Cu B.Cu) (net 5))
 (via micro (at 132.800002 391.000006) (size 0.300000) (drill 0.100000) (layers F.Cu B.Cu) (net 5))
 (via micro (at 131.700002 390.700006) (size 0.300000) (drill 0.100000) (layers F.Cu B.Cu) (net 5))
 (via micro (at 129.600002 390.700006) (size 0.300000) (drill 0.100000) (layers F.Cu B.Cu) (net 5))
 (segment (start 135.300002 389.100006) (end 135.400002 389.000006) (width 0.250000) (layer F.Cu) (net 7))
 (segment (start 135.400002 389.000006) (end 135.900002 389.000006) (width 0.250000) (layer F.Cu) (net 7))
 (segment (start 135.900002 389.000006) (end 136.700002 388.200006) (width 0.250000) (layer F.Cu) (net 7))
 (segment (start 136.700002 388.200006) (end 136.900002 388.000006) (width 0.250000) (layer B.Cu) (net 7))
 (segment (start 136.900002 388.000006) (end 136.900002 387.400006) (width 0.250000) (layer B.Cu) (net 7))
 (segment (start 136.900002 387.400006) (end 137.500002 386.800006) (width 0.250000) (layer B.Cu) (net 7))
 (segment (start 137.500002 386.800006) (end 137.100002 386.400006) (width 0.250000) (layer B.Cu) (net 7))
 (segment (start 137.100002 386.400006) (end 137.100002 386.100006) (width 0.250000) (layer F.Cu) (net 7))
 (segment (start 137.100002 386.100006) (end 136.800002 385.800006) (width 0.250000) (layer F.Cu) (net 7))
 (segment (start 136.800002 385.800006) (end 132.900002 385.800006) (width 0.250000) (layer F.Cu) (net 7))
 (segment (start 132.900002 385.800006) (end 132.800002 385.900006) (width 0.250000) (layer F.Cu) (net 7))
 (segment (start 132.800002 385.900006) (end 132.300002 385.900006) (width 0.250000) (layer F.Cu) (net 7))
 (segment (start 132.300002 385.900006) (end 132.200002 385.900006) (width 0.250000) (layer B.Cu) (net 7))
 (segment (start 132.200002 385.900006) (end 131.400002 385.100006) (width 0.250000) (layer B.Cu) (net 7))
 (segment (start 131.400002 385.100006) (end 131.400002 385.000006) (width 0.250000) (layer B.Cu) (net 7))
 (segment (start 131.400002 385.000006) (end 131.200002 384.800006) (width 0.250000) (layer B.Cu) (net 7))
 (segment (start 131.200002 384.800006) (end 130.600002 384.800006) (width 0.250000) (layer B.Cu) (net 7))
 (segment (start 130.600002 384.800006) (end 130.400002 385.000006) (width 0.250000) (layer B.Cu) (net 7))
 (segment (start 130.400002 385.000006) (end 130.400002 385.600006) (width 0.250000) (layer B.Cu) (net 7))
 (segment (start 130.400002 385.600006) (end 132.400002 387.600006) (width 0.250000) (layer B.Cu) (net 7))
 (segment (start 132.400002 387.600006) (end 131.900002 387.600006) (width 0.250000) (layer F.Cu) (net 7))
 (via micro (at 136.700002 388.200006) (size 0.300000) (drill 0.100000) (layers F.Cu B.Cu) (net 7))
 (via micro (at 137.100002 386.400006) (size 0.300000) (drill 0.100000) (layers F.Cu B.Cu) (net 7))
 (via micro (at 132.300002 385.900006) (size 0.300000) (drill 0.100000) (layers F.Cu B.Cu) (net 7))
 (via micro (at 132.400002 387.600006) (size 0.300000) (drill 0.100000) (layers F.Cu B.Cu) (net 7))
 (segment (start 131.600002 386.000006) (end 131.800002 386.000006) (width 0.250000) (layer F.Cu) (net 6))
 (segment (start 131.800002 386.000006) (end 132.200002 386.400006) (width 0.250000) (layer F.Cu) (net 6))
 (segment (start 132.200002 386.400006) (end 132.700002 386.400006) (width 0.250000) (layer B.Cu) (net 6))
 (segment (start 132.700002 386.400006) (end 133.500002 385.600006) (width 0.250000) (layer B.Cu) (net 6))
 (segment (start 133.500002 385.600006) (end 135.100002 385.600006) (width 0.250000) (layer B.Cu) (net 6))
 (segment (start 135.100002 385.600006) (end 135.900002 386.400006) (width 0.250000) (layer B.Cu) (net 6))
 (segment (start 135.900002 386.400006) (end 135.900002 386.500006) (width 0.250000) (layer B.Cu) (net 6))
 (segment (start 135.900002 386.500006) (end 135.700002 386.700006) (width 0.250000) (layer B.Cu) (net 6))
 (segment (start 135.700002 386.700006) (end 135.800002 386.700006) (width 0.250000) (layer F.Cu) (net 6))
 (segment (start 135.800002 386.700006) (end 135.900002 386.600006) (width 0.250000) (layer F.Cu) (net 6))
 (segment (start 135.900002 386.600006) (end 136.000002 386.600006) (width 0.250000) (layer F.Cu) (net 6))
 (segment (start 136.000002 386.600006) (end 136.200002 386.800006) (width 0.250000) (layer F.Cu) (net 6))
 (via micro (at 132.200002 386.400006) (size 0.300000) (drill 0.100000) (layers F.Cu B.Cu) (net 6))
 (via micro (at 135.700002 386.700006) (size 0.300000) (drill 0.100000) (layers F.Cu B.Cu) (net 6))
 (segment (start 130.400002 391.700006) (end 130.500002 391.600006) (width 0.250000) (layer F.Cu) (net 3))
 (segment (start 130.500002 391.600006) (end 130.500002 391.500006) (width 0.250000) (layer F.Cu) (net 3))
 (segment (start 130.500002 391.500006) (end 130.800002 391.200006) (width 0.250000) (layer F.Cu) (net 3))
 (segment (start 130.800002 391.200006) (end 129.300002 391.200006) (width 0.250000) (layer B.Cu) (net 3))
 (segment (start 129.300002 391.200006) (end 129.100002 391.000006) (width 0.250000) (layer B.Cu) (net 3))
 (segment (start 129.100002 391.000006) (end 129.100002 390.400006) (width 0.250000) (layer B.Cu) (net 3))
 (segment (start 129.100002 390.400006) (end 129.300002 390.200006) (width 0.250000) (layer B.Cu) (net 3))
 (segment (start 129.300002 390.200006) (end 130.200002 390.200006) (width 0.250000) (layer B.Cu) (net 3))
 (segment (start 130.200002 390.200006) (end 132.300002 388.100006) (width 0.250000) (layer B.Cu) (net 3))
 (segment (start 132.300002 388.100006) (end 132.600002 388.100006) (width 0.250000) (layer F.Cu) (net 3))
 (segment (start 132.600002 388.100006) (end 132.900002 387.800006) (width 0.250000) (layer F.Cu) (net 3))
 (segment (start 132.900002 387.800006) (end 132.900002 387.700006) (width 0.250000) (layer F.Cu) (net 3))
 (segment (start 132.900002 387.700006) (end 133.300002 387.300006) (width 0.250000) (layer F.Cu) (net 3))
 (segment (start 133.300002 387.300006) (end 133.400002 387.300006) (width 0.250000) (layer F.Cu) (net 3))
 (segment (start 133.400002 387.300006) (end 133.500002 387.200006) (width 0.250000) (layer F.Cu) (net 3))
 (segment (start 133.500002 387.200006) (end 133.200002 386.900006) (width 0.250000) (layer B.Cu) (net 3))
 (segment (start 133.200002 386.900006) (end 133.200002 386.700006) (width 0.250000) (layer B.Cu) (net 3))
 (segment (start 133.200002 386.700006) (end 134.000002 385.900006) (width 0.250000) (layer B.Cu) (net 3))
 (segment (start 134.000002 385.900006) (end 134.000002 385.500006) (width 0.250000) (layer B.Cu) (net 3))
 (segment (start 134.000002 385.500006) (end 133.800002 385.300006) (width 0.250000) (layer F.Cu) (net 3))
 (segment (start 133.800002 385.300006) (end 133.200002 385.300006) (width 0.250000) (layer F.Cu) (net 3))
 (via micro (at 130.800002 391.200006) (size 0.300000) (drill 0.100000) (layers F.Cu B.Cu) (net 3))
 (via micro (at 132.300002 388.100006) (size 0.300000) (drill 0.100000) (layers F.Cu B.Cu) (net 3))
 (via micro (at 133.500002 387.200006) (size 0.300000) (drill 0.100000) (layers F.Cu B.Cu) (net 3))
 (via micro (at 134.000002 385.500006) (size 0.300000) (drill 0.100000) (layers F.Cu B.Cu) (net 3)))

